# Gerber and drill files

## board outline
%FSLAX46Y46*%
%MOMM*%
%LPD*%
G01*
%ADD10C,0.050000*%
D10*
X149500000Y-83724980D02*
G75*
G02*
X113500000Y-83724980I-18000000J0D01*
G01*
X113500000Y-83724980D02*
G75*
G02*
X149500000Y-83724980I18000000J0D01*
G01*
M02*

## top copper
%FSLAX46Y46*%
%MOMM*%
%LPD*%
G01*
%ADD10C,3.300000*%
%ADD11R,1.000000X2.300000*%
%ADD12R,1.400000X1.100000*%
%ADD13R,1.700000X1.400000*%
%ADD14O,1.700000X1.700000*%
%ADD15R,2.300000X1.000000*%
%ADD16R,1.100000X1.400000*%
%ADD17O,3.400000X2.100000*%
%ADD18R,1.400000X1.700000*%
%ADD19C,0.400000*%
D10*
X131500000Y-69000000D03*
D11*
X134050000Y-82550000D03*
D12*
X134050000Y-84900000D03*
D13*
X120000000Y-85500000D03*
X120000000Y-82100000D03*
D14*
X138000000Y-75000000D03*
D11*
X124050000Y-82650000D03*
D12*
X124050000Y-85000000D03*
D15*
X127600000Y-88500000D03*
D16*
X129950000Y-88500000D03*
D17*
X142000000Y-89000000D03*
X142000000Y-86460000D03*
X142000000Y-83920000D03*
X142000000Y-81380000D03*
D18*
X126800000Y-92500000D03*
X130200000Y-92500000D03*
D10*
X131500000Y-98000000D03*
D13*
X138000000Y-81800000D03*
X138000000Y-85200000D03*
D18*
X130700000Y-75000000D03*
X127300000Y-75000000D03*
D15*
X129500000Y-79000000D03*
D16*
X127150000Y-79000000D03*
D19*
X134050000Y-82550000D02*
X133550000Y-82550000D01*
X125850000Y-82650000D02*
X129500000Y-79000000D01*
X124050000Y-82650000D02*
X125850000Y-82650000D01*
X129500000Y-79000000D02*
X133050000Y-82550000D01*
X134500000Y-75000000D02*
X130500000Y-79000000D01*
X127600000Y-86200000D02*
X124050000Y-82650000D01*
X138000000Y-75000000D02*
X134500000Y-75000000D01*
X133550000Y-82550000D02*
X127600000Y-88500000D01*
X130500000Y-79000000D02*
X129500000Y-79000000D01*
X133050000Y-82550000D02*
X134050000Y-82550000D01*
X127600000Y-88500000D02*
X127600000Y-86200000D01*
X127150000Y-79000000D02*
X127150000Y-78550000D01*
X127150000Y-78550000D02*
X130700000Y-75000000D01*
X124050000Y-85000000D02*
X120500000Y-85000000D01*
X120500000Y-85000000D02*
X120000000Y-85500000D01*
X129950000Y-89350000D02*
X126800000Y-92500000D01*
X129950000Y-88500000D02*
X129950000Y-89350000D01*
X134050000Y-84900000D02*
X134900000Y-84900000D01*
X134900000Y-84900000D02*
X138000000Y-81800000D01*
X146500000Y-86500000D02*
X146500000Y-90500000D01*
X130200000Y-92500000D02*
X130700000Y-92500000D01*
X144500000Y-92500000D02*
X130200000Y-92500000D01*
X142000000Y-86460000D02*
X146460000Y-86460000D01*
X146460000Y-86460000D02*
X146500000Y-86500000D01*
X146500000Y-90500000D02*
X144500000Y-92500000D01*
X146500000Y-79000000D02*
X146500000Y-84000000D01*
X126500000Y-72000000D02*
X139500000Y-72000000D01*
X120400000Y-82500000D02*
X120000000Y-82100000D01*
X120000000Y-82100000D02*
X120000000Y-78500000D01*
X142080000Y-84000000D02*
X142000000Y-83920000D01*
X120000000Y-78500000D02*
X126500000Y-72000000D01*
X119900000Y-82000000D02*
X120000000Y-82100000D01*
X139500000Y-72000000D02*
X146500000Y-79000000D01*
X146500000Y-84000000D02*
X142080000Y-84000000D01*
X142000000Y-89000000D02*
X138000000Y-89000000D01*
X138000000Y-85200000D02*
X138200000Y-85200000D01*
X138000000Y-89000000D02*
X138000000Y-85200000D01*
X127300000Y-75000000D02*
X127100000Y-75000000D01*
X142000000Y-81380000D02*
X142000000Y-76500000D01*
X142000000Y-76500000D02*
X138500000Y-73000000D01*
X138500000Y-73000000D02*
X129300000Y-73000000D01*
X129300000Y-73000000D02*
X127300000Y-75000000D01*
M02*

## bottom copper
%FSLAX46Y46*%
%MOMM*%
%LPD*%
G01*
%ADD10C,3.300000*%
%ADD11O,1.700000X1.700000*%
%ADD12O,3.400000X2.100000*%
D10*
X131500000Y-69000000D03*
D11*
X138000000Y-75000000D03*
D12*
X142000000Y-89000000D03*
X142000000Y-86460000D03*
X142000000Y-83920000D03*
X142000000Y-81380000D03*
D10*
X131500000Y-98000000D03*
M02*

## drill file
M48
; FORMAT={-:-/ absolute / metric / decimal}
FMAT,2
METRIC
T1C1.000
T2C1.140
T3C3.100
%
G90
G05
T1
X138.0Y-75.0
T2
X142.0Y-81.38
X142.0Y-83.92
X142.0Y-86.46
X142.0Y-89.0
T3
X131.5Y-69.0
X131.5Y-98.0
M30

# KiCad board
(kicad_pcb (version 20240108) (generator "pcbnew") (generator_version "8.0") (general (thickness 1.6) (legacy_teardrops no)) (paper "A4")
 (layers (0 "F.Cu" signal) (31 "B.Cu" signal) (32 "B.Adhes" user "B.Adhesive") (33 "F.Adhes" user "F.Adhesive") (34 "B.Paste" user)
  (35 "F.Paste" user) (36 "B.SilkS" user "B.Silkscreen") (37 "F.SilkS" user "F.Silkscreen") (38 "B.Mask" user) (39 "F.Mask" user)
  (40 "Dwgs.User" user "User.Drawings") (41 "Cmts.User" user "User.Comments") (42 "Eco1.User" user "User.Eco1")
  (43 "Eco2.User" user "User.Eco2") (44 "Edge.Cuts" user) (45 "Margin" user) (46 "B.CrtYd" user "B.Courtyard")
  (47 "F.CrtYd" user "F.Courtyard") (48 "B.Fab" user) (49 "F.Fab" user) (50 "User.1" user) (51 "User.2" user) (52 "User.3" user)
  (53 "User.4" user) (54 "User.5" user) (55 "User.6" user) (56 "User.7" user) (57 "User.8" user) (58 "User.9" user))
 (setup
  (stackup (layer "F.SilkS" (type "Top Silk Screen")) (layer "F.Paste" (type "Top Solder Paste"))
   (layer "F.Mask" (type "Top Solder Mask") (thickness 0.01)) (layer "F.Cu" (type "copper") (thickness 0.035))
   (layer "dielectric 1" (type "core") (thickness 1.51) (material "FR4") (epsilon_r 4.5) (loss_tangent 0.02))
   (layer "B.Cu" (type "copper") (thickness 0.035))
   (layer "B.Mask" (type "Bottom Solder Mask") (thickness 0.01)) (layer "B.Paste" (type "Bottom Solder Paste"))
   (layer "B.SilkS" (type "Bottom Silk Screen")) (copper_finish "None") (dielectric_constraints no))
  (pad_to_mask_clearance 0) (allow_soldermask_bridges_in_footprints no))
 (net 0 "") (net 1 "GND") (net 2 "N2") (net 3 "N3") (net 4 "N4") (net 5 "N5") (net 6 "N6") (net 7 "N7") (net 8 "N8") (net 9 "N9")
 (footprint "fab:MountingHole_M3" (layer "F.Cu") (at 131.5 69)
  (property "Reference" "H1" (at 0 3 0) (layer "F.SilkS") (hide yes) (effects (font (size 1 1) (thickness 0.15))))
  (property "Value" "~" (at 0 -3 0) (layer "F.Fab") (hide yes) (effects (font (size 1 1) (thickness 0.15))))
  (pad "" thru_hole circle (at 0 0) (size 3.3 3.3) (drill 3.1) (layers "*.Cu" "*.Mask") (remove_unused_layers no)))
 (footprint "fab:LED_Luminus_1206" (layer "F.Cu") (at 134.05 83.5 90)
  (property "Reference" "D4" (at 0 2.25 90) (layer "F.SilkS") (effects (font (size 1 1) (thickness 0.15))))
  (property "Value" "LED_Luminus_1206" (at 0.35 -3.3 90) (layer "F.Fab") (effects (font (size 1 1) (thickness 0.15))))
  (pad "1" smd rect (at 0.95 0 90) (size 2.3 1) (layers "F.Cu" "F.Paste" "F.Mask") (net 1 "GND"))
  (pad "2" smd rect (at -1.4 0 90) (size 1.1 1.4) (layers "F.Cu" "F.Paste" "F.Mask") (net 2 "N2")))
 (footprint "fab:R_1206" (layer "F.Cu") (at 120 83.8 90)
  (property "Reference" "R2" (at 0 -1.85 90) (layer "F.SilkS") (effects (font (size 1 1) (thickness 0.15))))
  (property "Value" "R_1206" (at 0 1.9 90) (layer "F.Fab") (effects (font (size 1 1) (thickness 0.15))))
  (pad "1" smd rect (at -1.7 0 90) (size 1.4 1.7) (layers "F.Cu" "F.Paste" "F.Mask") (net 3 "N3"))
  (pad "2" smd rect (at 1.7 0 90) (size 1.4 1.7) (layers "F.Cu" "F.Paste" "F.Mask") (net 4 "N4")))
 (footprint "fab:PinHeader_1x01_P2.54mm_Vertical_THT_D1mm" (layer "F.Cu") (at 138 75)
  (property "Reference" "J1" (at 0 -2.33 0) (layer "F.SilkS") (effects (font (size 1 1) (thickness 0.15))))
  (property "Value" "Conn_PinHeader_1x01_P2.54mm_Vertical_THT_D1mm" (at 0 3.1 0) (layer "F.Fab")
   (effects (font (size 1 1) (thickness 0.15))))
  (pad "1" thru_hole oval (at 0 0) (size 1.7 1.7) (drill 1) (layers "*.Cu" "*.Mask") (remove_unused_layers no) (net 1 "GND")))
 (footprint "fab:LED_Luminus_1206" (layer "F.Cu") (at 124.05 83.6 90)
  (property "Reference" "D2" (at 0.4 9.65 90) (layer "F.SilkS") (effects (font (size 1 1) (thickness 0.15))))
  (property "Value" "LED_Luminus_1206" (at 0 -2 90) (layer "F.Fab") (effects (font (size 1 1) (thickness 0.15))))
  (pad "1" smd rect (at 0.95 0 90) (size 2.3 1) (layers "F.Cu" "F.Paste" "F.Mask") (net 1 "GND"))
  (pad "2" smd rect (at -1.4 0 90) (size 1.1 1.4) (layers "F.Cu" "F.Paste" "F.Mask") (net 3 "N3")))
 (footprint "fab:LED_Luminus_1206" (layer "F.Cu") (at 128.55 88.5 180)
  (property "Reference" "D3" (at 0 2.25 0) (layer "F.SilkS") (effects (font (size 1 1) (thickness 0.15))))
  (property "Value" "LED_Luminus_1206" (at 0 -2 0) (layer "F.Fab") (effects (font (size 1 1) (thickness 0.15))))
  (pad "1" smd rect (at 0.95 0 180) (size 2.3 1) (layers "F.Cu" "F.Paste" "F.Mask") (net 1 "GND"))
  (pad "2" smd rect (at -1.4 0 180) (size 1.1 1.4) (layers "F.Cu" "F.Paste" "F.Mask") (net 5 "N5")))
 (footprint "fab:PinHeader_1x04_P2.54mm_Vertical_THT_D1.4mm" (layer "F.Cu") (at 142 89 180)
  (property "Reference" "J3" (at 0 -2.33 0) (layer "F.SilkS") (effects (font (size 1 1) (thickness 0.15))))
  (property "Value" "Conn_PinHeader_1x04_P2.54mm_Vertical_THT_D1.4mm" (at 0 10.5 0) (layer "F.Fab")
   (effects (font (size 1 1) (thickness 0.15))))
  (pad "1" thru_hole oval (at 0 0 180) (size 3.4 2.1) (drill 1.14) (layers "*.Cu" "*.Mask") (remove_unused_layers no) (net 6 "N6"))
  (pad "2" thru_hole oval (at 0 2.54 180) (size 3.4 2.1) (drill 1.14) (layers "*.Cu" "*.Mask") (remove_unused_layers no) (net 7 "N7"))
  (pad "3" thru_hole oval (at 0 5.08 180) (size 3.4 2.1) (drill 1.14) (layers "*.Cu" "*.Mask") (remove_unused_layers no) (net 4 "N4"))
  (pad "4" thru_hole oval (at 0 7.62 180) (size 3.4 2.1) (drill 1.14) (layers "*.Cu" "*.Mask") (remove_unused_layers no) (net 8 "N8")))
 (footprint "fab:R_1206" (layer "F.Cu") (at 128.5 92.5)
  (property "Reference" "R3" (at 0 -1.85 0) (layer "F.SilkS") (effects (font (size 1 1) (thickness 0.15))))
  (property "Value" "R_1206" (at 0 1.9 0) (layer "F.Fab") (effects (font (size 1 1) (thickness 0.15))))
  (pad "1" smd rect (at -1.7 0) (size 1.4 1.7) (layers "F.Cu" "F.Paste" "F.Mask") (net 5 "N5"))
  (pad "2" smd rect (at 1.7 0) (size 1.4 1.7) (layers "F.Cu" "F.Paste" "F.Mask") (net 7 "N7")))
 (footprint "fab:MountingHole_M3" (layer "F.Cu") (at 131.5 98)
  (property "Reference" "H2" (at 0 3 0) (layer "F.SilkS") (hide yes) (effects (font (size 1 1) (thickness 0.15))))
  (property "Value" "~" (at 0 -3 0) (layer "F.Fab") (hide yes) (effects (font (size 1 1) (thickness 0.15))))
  (pad "" thru_hole circle (at 0 0) (size 3.3 3.3) (drill 3.1) (layers "*.Cu" "*.Mask") (remove_unused_layers no)))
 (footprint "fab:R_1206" (layer "F.Cu") (at 138 83.5 -90)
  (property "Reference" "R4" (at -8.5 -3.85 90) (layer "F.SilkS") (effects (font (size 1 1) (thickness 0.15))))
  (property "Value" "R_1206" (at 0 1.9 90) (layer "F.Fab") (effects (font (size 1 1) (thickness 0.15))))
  (pad "1" smd rect (at -1.7 0 270) (size 1.4 1.7) (layers "F.Cu" "F.Paste" "F.Mask") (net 2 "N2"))
  (pad "2" smd rect (at 1.7 0 270) (size 1.4 1.7) (layers "F.Cu" "F.Paste" "F.Mask") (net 6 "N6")))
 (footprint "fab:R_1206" (layer "F.Cu") (at 129 75 180)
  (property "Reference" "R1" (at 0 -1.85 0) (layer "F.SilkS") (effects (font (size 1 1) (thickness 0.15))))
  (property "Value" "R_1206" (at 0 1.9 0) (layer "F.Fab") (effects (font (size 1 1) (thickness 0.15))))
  (pad "1" smd rect (at -1.7 0 180) (size 1.4 1.7) (layers "F.Cu" "F.Paste" "F.Mask") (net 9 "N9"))
  (pad "2" smd rect (at 1.7 0 180) (size 1.4 1.7) (layers "F.Cu" "F.Paste" "F.Mask") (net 8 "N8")))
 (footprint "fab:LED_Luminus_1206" (layer "F.Cu") (at 128.55 79)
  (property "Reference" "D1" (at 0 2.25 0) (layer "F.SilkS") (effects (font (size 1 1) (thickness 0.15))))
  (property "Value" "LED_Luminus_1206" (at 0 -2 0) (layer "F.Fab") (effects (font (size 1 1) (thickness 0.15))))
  (pad "1" smd rect (at 0.95 0) (size 2.3 1) (layers "F.Cu" "F.Paste" "F.Mask") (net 1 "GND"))
  (pad "2" smd rect (at -1.4 0) (size 1.1 1.4) (layers "F.Cu" "F.Paste" "F.Mask") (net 9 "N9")))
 (gr_circle (center 131.5 83.72498) (end 149.5 83.72498) (stroke (width 0.05) (type default)) (fill none) (layer "Edge.Cuts"))
 (segment (start 134.05 82.55) (end 133.55 82.55) (width 0.4) (layer "F.Cu") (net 1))
 (segment (start 125.85 82.65) (end 129.5 79) (width 0.4) (layer "F.Cu") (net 1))
 (segment (start 124.05 82.65) (end 125.85 82.65) (width 0.4) (layer "F.Cu") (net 1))
 (segment (start 129.5 79) (end 133.05 82.55) (width 0.4) (layer "F.Cu") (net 1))
 (segment (start 134.5 75) (end 130.5 79) (width 0.4) (layer "F.Cu") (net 1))
 (segment (start 127.6 86.2) (end 124.05 82.65) (width 0.4) (layer "F.Cu") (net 1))
 (segment (start 138 75) (end 134.5 75) (width 0.4) (layer "F.Cu") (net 1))
 (segment (start 133.55 82.55) (end 127.6 88.5) (width 0.4) (layer "F.Cu") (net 1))
 (segment (start 130.5 79) (end 129.5 79) (width 0.4) (layer "F.Cu") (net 1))
 (segment (start 133.05 82.55) (end 134.05 82.55) (width 0.4) (layer "F.Cu") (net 1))
 (segment (start 127.6 88.5) (end 127.6 86.2) (width 0.4) (layer "F.Cu") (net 1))
 (segment (start 127.15 79) (end 127.15 78.55) (width 0.4) (layer "F.Cu") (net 9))
 (segment (start 127.15 78.55) (end 130.7 75) (width 0.4) (layer "F.Cu") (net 9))
 (segment (start 124.05 85) (end 120.5 85) (width 0.4) (layer "F.Cu") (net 3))
 (segment (start 120.5 85) (end 120 85.5) (width 0.4) (layer "F.Cu") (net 3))
 (segment (start 129.95 89.35) (end 126.8 92.5) (width 0.4) (layer "F.Cu") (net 5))
 (segment (start 129.95 88.5) (end 129.95 89.35) (width 0.4) (layer "F.Cu") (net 5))
 (segment (start 134.05 84.9) (end 134.9 84.9) (width 0.4) (layer "F.Cu") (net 2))
 (segment (start 134.9 84.9) (end 138 81.8) (width 0.4) (layer "F.Cu") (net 2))
 (segment (start 146.5 86.5) (end 146.5 90.5) (width 0.4) (layer "F.Cu") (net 7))
 (segment (start 130.2 92.5) (end 130.7 92.5) (width 0.4) (layer "F.Cu") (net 7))
 (segment (start 144.5 92.5) (end 130.2 92.5) (width 0.4) (layer "F.Cu") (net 7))
 (segment (start 142 86.46) (end 146.46 86.46) (width 0.4) (layer "F.Cu") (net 7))
 (segment (start 146.46 86.46) (end 146.5 86.5) (width 0.4) (layer "F.Cu") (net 7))
 (segment (start 146.5 90.5) (end 144.5 92.5) (width 0.4) (layer "F.Cu") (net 7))
 (segment (start 146.5 79) (end 146.5 84) (width 0.4) (layer "F.Cu") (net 4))
 (segment (start 126.5 72) (end 139.5 72) (width 0.4) (layer "F.Cu") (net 4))
 (segment (start 120.4 82.5) (end 120 82.1) (width 0.4) (layer "F.Cu") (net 4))
 (segment (start 120 82.1) (end 120 78.5) (width 0.4) (layer "F.Cu") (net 4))
 (segment (start 142.08 84) (end 142 83.92) (width 0.4) (layer "F.Cu") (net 4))
 (segment (start 120 78.5) (end 126.5 72) (width 0.4) (layer "F.Cu") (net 4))
 (segment (start 119.9 82) (end 120 82.1) (width 0.4) (layer "F.Cu") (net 4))
 (segment (start 139.5 72) (end 146.5 79) (width 0.4) (layer "F.Cu") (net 4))
 (segment (start 146.5 84) (end 142.08 84) (width 0.4) (layer "F.Cu") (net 4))
 (segment (start 142 89) (end 138 89) (width 0.4) (layer "F.Cu") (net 6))
 (segment (start 138 85.2) (end 138.2 85.2) (width 0.4) (layer "F.Cu") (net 6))
 (segment (start 138 89) (end 138 85.2) (width 0.4) (layer "F.Cu") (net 6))
 (segment (start 127.3 75) (end 127.1 75) (width 0.4) (layer "F.Cu") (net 8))
 (segment (start 142 81.38) (end 142 76.5) (width 0.4) (layer "F.Cu") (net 8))
 (segment (start 142 76.5) (end 138.5 73) (width 0.4) (layer "F.Cu") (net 8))
 (segment (start 138.5 73) (end 129.3 73) (width 0.4) (layer "F.Cu") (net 8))
 (segment (start 129.3 73) (end 127.3 75) (width 0.4) (layer "F.Cu") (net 8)))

